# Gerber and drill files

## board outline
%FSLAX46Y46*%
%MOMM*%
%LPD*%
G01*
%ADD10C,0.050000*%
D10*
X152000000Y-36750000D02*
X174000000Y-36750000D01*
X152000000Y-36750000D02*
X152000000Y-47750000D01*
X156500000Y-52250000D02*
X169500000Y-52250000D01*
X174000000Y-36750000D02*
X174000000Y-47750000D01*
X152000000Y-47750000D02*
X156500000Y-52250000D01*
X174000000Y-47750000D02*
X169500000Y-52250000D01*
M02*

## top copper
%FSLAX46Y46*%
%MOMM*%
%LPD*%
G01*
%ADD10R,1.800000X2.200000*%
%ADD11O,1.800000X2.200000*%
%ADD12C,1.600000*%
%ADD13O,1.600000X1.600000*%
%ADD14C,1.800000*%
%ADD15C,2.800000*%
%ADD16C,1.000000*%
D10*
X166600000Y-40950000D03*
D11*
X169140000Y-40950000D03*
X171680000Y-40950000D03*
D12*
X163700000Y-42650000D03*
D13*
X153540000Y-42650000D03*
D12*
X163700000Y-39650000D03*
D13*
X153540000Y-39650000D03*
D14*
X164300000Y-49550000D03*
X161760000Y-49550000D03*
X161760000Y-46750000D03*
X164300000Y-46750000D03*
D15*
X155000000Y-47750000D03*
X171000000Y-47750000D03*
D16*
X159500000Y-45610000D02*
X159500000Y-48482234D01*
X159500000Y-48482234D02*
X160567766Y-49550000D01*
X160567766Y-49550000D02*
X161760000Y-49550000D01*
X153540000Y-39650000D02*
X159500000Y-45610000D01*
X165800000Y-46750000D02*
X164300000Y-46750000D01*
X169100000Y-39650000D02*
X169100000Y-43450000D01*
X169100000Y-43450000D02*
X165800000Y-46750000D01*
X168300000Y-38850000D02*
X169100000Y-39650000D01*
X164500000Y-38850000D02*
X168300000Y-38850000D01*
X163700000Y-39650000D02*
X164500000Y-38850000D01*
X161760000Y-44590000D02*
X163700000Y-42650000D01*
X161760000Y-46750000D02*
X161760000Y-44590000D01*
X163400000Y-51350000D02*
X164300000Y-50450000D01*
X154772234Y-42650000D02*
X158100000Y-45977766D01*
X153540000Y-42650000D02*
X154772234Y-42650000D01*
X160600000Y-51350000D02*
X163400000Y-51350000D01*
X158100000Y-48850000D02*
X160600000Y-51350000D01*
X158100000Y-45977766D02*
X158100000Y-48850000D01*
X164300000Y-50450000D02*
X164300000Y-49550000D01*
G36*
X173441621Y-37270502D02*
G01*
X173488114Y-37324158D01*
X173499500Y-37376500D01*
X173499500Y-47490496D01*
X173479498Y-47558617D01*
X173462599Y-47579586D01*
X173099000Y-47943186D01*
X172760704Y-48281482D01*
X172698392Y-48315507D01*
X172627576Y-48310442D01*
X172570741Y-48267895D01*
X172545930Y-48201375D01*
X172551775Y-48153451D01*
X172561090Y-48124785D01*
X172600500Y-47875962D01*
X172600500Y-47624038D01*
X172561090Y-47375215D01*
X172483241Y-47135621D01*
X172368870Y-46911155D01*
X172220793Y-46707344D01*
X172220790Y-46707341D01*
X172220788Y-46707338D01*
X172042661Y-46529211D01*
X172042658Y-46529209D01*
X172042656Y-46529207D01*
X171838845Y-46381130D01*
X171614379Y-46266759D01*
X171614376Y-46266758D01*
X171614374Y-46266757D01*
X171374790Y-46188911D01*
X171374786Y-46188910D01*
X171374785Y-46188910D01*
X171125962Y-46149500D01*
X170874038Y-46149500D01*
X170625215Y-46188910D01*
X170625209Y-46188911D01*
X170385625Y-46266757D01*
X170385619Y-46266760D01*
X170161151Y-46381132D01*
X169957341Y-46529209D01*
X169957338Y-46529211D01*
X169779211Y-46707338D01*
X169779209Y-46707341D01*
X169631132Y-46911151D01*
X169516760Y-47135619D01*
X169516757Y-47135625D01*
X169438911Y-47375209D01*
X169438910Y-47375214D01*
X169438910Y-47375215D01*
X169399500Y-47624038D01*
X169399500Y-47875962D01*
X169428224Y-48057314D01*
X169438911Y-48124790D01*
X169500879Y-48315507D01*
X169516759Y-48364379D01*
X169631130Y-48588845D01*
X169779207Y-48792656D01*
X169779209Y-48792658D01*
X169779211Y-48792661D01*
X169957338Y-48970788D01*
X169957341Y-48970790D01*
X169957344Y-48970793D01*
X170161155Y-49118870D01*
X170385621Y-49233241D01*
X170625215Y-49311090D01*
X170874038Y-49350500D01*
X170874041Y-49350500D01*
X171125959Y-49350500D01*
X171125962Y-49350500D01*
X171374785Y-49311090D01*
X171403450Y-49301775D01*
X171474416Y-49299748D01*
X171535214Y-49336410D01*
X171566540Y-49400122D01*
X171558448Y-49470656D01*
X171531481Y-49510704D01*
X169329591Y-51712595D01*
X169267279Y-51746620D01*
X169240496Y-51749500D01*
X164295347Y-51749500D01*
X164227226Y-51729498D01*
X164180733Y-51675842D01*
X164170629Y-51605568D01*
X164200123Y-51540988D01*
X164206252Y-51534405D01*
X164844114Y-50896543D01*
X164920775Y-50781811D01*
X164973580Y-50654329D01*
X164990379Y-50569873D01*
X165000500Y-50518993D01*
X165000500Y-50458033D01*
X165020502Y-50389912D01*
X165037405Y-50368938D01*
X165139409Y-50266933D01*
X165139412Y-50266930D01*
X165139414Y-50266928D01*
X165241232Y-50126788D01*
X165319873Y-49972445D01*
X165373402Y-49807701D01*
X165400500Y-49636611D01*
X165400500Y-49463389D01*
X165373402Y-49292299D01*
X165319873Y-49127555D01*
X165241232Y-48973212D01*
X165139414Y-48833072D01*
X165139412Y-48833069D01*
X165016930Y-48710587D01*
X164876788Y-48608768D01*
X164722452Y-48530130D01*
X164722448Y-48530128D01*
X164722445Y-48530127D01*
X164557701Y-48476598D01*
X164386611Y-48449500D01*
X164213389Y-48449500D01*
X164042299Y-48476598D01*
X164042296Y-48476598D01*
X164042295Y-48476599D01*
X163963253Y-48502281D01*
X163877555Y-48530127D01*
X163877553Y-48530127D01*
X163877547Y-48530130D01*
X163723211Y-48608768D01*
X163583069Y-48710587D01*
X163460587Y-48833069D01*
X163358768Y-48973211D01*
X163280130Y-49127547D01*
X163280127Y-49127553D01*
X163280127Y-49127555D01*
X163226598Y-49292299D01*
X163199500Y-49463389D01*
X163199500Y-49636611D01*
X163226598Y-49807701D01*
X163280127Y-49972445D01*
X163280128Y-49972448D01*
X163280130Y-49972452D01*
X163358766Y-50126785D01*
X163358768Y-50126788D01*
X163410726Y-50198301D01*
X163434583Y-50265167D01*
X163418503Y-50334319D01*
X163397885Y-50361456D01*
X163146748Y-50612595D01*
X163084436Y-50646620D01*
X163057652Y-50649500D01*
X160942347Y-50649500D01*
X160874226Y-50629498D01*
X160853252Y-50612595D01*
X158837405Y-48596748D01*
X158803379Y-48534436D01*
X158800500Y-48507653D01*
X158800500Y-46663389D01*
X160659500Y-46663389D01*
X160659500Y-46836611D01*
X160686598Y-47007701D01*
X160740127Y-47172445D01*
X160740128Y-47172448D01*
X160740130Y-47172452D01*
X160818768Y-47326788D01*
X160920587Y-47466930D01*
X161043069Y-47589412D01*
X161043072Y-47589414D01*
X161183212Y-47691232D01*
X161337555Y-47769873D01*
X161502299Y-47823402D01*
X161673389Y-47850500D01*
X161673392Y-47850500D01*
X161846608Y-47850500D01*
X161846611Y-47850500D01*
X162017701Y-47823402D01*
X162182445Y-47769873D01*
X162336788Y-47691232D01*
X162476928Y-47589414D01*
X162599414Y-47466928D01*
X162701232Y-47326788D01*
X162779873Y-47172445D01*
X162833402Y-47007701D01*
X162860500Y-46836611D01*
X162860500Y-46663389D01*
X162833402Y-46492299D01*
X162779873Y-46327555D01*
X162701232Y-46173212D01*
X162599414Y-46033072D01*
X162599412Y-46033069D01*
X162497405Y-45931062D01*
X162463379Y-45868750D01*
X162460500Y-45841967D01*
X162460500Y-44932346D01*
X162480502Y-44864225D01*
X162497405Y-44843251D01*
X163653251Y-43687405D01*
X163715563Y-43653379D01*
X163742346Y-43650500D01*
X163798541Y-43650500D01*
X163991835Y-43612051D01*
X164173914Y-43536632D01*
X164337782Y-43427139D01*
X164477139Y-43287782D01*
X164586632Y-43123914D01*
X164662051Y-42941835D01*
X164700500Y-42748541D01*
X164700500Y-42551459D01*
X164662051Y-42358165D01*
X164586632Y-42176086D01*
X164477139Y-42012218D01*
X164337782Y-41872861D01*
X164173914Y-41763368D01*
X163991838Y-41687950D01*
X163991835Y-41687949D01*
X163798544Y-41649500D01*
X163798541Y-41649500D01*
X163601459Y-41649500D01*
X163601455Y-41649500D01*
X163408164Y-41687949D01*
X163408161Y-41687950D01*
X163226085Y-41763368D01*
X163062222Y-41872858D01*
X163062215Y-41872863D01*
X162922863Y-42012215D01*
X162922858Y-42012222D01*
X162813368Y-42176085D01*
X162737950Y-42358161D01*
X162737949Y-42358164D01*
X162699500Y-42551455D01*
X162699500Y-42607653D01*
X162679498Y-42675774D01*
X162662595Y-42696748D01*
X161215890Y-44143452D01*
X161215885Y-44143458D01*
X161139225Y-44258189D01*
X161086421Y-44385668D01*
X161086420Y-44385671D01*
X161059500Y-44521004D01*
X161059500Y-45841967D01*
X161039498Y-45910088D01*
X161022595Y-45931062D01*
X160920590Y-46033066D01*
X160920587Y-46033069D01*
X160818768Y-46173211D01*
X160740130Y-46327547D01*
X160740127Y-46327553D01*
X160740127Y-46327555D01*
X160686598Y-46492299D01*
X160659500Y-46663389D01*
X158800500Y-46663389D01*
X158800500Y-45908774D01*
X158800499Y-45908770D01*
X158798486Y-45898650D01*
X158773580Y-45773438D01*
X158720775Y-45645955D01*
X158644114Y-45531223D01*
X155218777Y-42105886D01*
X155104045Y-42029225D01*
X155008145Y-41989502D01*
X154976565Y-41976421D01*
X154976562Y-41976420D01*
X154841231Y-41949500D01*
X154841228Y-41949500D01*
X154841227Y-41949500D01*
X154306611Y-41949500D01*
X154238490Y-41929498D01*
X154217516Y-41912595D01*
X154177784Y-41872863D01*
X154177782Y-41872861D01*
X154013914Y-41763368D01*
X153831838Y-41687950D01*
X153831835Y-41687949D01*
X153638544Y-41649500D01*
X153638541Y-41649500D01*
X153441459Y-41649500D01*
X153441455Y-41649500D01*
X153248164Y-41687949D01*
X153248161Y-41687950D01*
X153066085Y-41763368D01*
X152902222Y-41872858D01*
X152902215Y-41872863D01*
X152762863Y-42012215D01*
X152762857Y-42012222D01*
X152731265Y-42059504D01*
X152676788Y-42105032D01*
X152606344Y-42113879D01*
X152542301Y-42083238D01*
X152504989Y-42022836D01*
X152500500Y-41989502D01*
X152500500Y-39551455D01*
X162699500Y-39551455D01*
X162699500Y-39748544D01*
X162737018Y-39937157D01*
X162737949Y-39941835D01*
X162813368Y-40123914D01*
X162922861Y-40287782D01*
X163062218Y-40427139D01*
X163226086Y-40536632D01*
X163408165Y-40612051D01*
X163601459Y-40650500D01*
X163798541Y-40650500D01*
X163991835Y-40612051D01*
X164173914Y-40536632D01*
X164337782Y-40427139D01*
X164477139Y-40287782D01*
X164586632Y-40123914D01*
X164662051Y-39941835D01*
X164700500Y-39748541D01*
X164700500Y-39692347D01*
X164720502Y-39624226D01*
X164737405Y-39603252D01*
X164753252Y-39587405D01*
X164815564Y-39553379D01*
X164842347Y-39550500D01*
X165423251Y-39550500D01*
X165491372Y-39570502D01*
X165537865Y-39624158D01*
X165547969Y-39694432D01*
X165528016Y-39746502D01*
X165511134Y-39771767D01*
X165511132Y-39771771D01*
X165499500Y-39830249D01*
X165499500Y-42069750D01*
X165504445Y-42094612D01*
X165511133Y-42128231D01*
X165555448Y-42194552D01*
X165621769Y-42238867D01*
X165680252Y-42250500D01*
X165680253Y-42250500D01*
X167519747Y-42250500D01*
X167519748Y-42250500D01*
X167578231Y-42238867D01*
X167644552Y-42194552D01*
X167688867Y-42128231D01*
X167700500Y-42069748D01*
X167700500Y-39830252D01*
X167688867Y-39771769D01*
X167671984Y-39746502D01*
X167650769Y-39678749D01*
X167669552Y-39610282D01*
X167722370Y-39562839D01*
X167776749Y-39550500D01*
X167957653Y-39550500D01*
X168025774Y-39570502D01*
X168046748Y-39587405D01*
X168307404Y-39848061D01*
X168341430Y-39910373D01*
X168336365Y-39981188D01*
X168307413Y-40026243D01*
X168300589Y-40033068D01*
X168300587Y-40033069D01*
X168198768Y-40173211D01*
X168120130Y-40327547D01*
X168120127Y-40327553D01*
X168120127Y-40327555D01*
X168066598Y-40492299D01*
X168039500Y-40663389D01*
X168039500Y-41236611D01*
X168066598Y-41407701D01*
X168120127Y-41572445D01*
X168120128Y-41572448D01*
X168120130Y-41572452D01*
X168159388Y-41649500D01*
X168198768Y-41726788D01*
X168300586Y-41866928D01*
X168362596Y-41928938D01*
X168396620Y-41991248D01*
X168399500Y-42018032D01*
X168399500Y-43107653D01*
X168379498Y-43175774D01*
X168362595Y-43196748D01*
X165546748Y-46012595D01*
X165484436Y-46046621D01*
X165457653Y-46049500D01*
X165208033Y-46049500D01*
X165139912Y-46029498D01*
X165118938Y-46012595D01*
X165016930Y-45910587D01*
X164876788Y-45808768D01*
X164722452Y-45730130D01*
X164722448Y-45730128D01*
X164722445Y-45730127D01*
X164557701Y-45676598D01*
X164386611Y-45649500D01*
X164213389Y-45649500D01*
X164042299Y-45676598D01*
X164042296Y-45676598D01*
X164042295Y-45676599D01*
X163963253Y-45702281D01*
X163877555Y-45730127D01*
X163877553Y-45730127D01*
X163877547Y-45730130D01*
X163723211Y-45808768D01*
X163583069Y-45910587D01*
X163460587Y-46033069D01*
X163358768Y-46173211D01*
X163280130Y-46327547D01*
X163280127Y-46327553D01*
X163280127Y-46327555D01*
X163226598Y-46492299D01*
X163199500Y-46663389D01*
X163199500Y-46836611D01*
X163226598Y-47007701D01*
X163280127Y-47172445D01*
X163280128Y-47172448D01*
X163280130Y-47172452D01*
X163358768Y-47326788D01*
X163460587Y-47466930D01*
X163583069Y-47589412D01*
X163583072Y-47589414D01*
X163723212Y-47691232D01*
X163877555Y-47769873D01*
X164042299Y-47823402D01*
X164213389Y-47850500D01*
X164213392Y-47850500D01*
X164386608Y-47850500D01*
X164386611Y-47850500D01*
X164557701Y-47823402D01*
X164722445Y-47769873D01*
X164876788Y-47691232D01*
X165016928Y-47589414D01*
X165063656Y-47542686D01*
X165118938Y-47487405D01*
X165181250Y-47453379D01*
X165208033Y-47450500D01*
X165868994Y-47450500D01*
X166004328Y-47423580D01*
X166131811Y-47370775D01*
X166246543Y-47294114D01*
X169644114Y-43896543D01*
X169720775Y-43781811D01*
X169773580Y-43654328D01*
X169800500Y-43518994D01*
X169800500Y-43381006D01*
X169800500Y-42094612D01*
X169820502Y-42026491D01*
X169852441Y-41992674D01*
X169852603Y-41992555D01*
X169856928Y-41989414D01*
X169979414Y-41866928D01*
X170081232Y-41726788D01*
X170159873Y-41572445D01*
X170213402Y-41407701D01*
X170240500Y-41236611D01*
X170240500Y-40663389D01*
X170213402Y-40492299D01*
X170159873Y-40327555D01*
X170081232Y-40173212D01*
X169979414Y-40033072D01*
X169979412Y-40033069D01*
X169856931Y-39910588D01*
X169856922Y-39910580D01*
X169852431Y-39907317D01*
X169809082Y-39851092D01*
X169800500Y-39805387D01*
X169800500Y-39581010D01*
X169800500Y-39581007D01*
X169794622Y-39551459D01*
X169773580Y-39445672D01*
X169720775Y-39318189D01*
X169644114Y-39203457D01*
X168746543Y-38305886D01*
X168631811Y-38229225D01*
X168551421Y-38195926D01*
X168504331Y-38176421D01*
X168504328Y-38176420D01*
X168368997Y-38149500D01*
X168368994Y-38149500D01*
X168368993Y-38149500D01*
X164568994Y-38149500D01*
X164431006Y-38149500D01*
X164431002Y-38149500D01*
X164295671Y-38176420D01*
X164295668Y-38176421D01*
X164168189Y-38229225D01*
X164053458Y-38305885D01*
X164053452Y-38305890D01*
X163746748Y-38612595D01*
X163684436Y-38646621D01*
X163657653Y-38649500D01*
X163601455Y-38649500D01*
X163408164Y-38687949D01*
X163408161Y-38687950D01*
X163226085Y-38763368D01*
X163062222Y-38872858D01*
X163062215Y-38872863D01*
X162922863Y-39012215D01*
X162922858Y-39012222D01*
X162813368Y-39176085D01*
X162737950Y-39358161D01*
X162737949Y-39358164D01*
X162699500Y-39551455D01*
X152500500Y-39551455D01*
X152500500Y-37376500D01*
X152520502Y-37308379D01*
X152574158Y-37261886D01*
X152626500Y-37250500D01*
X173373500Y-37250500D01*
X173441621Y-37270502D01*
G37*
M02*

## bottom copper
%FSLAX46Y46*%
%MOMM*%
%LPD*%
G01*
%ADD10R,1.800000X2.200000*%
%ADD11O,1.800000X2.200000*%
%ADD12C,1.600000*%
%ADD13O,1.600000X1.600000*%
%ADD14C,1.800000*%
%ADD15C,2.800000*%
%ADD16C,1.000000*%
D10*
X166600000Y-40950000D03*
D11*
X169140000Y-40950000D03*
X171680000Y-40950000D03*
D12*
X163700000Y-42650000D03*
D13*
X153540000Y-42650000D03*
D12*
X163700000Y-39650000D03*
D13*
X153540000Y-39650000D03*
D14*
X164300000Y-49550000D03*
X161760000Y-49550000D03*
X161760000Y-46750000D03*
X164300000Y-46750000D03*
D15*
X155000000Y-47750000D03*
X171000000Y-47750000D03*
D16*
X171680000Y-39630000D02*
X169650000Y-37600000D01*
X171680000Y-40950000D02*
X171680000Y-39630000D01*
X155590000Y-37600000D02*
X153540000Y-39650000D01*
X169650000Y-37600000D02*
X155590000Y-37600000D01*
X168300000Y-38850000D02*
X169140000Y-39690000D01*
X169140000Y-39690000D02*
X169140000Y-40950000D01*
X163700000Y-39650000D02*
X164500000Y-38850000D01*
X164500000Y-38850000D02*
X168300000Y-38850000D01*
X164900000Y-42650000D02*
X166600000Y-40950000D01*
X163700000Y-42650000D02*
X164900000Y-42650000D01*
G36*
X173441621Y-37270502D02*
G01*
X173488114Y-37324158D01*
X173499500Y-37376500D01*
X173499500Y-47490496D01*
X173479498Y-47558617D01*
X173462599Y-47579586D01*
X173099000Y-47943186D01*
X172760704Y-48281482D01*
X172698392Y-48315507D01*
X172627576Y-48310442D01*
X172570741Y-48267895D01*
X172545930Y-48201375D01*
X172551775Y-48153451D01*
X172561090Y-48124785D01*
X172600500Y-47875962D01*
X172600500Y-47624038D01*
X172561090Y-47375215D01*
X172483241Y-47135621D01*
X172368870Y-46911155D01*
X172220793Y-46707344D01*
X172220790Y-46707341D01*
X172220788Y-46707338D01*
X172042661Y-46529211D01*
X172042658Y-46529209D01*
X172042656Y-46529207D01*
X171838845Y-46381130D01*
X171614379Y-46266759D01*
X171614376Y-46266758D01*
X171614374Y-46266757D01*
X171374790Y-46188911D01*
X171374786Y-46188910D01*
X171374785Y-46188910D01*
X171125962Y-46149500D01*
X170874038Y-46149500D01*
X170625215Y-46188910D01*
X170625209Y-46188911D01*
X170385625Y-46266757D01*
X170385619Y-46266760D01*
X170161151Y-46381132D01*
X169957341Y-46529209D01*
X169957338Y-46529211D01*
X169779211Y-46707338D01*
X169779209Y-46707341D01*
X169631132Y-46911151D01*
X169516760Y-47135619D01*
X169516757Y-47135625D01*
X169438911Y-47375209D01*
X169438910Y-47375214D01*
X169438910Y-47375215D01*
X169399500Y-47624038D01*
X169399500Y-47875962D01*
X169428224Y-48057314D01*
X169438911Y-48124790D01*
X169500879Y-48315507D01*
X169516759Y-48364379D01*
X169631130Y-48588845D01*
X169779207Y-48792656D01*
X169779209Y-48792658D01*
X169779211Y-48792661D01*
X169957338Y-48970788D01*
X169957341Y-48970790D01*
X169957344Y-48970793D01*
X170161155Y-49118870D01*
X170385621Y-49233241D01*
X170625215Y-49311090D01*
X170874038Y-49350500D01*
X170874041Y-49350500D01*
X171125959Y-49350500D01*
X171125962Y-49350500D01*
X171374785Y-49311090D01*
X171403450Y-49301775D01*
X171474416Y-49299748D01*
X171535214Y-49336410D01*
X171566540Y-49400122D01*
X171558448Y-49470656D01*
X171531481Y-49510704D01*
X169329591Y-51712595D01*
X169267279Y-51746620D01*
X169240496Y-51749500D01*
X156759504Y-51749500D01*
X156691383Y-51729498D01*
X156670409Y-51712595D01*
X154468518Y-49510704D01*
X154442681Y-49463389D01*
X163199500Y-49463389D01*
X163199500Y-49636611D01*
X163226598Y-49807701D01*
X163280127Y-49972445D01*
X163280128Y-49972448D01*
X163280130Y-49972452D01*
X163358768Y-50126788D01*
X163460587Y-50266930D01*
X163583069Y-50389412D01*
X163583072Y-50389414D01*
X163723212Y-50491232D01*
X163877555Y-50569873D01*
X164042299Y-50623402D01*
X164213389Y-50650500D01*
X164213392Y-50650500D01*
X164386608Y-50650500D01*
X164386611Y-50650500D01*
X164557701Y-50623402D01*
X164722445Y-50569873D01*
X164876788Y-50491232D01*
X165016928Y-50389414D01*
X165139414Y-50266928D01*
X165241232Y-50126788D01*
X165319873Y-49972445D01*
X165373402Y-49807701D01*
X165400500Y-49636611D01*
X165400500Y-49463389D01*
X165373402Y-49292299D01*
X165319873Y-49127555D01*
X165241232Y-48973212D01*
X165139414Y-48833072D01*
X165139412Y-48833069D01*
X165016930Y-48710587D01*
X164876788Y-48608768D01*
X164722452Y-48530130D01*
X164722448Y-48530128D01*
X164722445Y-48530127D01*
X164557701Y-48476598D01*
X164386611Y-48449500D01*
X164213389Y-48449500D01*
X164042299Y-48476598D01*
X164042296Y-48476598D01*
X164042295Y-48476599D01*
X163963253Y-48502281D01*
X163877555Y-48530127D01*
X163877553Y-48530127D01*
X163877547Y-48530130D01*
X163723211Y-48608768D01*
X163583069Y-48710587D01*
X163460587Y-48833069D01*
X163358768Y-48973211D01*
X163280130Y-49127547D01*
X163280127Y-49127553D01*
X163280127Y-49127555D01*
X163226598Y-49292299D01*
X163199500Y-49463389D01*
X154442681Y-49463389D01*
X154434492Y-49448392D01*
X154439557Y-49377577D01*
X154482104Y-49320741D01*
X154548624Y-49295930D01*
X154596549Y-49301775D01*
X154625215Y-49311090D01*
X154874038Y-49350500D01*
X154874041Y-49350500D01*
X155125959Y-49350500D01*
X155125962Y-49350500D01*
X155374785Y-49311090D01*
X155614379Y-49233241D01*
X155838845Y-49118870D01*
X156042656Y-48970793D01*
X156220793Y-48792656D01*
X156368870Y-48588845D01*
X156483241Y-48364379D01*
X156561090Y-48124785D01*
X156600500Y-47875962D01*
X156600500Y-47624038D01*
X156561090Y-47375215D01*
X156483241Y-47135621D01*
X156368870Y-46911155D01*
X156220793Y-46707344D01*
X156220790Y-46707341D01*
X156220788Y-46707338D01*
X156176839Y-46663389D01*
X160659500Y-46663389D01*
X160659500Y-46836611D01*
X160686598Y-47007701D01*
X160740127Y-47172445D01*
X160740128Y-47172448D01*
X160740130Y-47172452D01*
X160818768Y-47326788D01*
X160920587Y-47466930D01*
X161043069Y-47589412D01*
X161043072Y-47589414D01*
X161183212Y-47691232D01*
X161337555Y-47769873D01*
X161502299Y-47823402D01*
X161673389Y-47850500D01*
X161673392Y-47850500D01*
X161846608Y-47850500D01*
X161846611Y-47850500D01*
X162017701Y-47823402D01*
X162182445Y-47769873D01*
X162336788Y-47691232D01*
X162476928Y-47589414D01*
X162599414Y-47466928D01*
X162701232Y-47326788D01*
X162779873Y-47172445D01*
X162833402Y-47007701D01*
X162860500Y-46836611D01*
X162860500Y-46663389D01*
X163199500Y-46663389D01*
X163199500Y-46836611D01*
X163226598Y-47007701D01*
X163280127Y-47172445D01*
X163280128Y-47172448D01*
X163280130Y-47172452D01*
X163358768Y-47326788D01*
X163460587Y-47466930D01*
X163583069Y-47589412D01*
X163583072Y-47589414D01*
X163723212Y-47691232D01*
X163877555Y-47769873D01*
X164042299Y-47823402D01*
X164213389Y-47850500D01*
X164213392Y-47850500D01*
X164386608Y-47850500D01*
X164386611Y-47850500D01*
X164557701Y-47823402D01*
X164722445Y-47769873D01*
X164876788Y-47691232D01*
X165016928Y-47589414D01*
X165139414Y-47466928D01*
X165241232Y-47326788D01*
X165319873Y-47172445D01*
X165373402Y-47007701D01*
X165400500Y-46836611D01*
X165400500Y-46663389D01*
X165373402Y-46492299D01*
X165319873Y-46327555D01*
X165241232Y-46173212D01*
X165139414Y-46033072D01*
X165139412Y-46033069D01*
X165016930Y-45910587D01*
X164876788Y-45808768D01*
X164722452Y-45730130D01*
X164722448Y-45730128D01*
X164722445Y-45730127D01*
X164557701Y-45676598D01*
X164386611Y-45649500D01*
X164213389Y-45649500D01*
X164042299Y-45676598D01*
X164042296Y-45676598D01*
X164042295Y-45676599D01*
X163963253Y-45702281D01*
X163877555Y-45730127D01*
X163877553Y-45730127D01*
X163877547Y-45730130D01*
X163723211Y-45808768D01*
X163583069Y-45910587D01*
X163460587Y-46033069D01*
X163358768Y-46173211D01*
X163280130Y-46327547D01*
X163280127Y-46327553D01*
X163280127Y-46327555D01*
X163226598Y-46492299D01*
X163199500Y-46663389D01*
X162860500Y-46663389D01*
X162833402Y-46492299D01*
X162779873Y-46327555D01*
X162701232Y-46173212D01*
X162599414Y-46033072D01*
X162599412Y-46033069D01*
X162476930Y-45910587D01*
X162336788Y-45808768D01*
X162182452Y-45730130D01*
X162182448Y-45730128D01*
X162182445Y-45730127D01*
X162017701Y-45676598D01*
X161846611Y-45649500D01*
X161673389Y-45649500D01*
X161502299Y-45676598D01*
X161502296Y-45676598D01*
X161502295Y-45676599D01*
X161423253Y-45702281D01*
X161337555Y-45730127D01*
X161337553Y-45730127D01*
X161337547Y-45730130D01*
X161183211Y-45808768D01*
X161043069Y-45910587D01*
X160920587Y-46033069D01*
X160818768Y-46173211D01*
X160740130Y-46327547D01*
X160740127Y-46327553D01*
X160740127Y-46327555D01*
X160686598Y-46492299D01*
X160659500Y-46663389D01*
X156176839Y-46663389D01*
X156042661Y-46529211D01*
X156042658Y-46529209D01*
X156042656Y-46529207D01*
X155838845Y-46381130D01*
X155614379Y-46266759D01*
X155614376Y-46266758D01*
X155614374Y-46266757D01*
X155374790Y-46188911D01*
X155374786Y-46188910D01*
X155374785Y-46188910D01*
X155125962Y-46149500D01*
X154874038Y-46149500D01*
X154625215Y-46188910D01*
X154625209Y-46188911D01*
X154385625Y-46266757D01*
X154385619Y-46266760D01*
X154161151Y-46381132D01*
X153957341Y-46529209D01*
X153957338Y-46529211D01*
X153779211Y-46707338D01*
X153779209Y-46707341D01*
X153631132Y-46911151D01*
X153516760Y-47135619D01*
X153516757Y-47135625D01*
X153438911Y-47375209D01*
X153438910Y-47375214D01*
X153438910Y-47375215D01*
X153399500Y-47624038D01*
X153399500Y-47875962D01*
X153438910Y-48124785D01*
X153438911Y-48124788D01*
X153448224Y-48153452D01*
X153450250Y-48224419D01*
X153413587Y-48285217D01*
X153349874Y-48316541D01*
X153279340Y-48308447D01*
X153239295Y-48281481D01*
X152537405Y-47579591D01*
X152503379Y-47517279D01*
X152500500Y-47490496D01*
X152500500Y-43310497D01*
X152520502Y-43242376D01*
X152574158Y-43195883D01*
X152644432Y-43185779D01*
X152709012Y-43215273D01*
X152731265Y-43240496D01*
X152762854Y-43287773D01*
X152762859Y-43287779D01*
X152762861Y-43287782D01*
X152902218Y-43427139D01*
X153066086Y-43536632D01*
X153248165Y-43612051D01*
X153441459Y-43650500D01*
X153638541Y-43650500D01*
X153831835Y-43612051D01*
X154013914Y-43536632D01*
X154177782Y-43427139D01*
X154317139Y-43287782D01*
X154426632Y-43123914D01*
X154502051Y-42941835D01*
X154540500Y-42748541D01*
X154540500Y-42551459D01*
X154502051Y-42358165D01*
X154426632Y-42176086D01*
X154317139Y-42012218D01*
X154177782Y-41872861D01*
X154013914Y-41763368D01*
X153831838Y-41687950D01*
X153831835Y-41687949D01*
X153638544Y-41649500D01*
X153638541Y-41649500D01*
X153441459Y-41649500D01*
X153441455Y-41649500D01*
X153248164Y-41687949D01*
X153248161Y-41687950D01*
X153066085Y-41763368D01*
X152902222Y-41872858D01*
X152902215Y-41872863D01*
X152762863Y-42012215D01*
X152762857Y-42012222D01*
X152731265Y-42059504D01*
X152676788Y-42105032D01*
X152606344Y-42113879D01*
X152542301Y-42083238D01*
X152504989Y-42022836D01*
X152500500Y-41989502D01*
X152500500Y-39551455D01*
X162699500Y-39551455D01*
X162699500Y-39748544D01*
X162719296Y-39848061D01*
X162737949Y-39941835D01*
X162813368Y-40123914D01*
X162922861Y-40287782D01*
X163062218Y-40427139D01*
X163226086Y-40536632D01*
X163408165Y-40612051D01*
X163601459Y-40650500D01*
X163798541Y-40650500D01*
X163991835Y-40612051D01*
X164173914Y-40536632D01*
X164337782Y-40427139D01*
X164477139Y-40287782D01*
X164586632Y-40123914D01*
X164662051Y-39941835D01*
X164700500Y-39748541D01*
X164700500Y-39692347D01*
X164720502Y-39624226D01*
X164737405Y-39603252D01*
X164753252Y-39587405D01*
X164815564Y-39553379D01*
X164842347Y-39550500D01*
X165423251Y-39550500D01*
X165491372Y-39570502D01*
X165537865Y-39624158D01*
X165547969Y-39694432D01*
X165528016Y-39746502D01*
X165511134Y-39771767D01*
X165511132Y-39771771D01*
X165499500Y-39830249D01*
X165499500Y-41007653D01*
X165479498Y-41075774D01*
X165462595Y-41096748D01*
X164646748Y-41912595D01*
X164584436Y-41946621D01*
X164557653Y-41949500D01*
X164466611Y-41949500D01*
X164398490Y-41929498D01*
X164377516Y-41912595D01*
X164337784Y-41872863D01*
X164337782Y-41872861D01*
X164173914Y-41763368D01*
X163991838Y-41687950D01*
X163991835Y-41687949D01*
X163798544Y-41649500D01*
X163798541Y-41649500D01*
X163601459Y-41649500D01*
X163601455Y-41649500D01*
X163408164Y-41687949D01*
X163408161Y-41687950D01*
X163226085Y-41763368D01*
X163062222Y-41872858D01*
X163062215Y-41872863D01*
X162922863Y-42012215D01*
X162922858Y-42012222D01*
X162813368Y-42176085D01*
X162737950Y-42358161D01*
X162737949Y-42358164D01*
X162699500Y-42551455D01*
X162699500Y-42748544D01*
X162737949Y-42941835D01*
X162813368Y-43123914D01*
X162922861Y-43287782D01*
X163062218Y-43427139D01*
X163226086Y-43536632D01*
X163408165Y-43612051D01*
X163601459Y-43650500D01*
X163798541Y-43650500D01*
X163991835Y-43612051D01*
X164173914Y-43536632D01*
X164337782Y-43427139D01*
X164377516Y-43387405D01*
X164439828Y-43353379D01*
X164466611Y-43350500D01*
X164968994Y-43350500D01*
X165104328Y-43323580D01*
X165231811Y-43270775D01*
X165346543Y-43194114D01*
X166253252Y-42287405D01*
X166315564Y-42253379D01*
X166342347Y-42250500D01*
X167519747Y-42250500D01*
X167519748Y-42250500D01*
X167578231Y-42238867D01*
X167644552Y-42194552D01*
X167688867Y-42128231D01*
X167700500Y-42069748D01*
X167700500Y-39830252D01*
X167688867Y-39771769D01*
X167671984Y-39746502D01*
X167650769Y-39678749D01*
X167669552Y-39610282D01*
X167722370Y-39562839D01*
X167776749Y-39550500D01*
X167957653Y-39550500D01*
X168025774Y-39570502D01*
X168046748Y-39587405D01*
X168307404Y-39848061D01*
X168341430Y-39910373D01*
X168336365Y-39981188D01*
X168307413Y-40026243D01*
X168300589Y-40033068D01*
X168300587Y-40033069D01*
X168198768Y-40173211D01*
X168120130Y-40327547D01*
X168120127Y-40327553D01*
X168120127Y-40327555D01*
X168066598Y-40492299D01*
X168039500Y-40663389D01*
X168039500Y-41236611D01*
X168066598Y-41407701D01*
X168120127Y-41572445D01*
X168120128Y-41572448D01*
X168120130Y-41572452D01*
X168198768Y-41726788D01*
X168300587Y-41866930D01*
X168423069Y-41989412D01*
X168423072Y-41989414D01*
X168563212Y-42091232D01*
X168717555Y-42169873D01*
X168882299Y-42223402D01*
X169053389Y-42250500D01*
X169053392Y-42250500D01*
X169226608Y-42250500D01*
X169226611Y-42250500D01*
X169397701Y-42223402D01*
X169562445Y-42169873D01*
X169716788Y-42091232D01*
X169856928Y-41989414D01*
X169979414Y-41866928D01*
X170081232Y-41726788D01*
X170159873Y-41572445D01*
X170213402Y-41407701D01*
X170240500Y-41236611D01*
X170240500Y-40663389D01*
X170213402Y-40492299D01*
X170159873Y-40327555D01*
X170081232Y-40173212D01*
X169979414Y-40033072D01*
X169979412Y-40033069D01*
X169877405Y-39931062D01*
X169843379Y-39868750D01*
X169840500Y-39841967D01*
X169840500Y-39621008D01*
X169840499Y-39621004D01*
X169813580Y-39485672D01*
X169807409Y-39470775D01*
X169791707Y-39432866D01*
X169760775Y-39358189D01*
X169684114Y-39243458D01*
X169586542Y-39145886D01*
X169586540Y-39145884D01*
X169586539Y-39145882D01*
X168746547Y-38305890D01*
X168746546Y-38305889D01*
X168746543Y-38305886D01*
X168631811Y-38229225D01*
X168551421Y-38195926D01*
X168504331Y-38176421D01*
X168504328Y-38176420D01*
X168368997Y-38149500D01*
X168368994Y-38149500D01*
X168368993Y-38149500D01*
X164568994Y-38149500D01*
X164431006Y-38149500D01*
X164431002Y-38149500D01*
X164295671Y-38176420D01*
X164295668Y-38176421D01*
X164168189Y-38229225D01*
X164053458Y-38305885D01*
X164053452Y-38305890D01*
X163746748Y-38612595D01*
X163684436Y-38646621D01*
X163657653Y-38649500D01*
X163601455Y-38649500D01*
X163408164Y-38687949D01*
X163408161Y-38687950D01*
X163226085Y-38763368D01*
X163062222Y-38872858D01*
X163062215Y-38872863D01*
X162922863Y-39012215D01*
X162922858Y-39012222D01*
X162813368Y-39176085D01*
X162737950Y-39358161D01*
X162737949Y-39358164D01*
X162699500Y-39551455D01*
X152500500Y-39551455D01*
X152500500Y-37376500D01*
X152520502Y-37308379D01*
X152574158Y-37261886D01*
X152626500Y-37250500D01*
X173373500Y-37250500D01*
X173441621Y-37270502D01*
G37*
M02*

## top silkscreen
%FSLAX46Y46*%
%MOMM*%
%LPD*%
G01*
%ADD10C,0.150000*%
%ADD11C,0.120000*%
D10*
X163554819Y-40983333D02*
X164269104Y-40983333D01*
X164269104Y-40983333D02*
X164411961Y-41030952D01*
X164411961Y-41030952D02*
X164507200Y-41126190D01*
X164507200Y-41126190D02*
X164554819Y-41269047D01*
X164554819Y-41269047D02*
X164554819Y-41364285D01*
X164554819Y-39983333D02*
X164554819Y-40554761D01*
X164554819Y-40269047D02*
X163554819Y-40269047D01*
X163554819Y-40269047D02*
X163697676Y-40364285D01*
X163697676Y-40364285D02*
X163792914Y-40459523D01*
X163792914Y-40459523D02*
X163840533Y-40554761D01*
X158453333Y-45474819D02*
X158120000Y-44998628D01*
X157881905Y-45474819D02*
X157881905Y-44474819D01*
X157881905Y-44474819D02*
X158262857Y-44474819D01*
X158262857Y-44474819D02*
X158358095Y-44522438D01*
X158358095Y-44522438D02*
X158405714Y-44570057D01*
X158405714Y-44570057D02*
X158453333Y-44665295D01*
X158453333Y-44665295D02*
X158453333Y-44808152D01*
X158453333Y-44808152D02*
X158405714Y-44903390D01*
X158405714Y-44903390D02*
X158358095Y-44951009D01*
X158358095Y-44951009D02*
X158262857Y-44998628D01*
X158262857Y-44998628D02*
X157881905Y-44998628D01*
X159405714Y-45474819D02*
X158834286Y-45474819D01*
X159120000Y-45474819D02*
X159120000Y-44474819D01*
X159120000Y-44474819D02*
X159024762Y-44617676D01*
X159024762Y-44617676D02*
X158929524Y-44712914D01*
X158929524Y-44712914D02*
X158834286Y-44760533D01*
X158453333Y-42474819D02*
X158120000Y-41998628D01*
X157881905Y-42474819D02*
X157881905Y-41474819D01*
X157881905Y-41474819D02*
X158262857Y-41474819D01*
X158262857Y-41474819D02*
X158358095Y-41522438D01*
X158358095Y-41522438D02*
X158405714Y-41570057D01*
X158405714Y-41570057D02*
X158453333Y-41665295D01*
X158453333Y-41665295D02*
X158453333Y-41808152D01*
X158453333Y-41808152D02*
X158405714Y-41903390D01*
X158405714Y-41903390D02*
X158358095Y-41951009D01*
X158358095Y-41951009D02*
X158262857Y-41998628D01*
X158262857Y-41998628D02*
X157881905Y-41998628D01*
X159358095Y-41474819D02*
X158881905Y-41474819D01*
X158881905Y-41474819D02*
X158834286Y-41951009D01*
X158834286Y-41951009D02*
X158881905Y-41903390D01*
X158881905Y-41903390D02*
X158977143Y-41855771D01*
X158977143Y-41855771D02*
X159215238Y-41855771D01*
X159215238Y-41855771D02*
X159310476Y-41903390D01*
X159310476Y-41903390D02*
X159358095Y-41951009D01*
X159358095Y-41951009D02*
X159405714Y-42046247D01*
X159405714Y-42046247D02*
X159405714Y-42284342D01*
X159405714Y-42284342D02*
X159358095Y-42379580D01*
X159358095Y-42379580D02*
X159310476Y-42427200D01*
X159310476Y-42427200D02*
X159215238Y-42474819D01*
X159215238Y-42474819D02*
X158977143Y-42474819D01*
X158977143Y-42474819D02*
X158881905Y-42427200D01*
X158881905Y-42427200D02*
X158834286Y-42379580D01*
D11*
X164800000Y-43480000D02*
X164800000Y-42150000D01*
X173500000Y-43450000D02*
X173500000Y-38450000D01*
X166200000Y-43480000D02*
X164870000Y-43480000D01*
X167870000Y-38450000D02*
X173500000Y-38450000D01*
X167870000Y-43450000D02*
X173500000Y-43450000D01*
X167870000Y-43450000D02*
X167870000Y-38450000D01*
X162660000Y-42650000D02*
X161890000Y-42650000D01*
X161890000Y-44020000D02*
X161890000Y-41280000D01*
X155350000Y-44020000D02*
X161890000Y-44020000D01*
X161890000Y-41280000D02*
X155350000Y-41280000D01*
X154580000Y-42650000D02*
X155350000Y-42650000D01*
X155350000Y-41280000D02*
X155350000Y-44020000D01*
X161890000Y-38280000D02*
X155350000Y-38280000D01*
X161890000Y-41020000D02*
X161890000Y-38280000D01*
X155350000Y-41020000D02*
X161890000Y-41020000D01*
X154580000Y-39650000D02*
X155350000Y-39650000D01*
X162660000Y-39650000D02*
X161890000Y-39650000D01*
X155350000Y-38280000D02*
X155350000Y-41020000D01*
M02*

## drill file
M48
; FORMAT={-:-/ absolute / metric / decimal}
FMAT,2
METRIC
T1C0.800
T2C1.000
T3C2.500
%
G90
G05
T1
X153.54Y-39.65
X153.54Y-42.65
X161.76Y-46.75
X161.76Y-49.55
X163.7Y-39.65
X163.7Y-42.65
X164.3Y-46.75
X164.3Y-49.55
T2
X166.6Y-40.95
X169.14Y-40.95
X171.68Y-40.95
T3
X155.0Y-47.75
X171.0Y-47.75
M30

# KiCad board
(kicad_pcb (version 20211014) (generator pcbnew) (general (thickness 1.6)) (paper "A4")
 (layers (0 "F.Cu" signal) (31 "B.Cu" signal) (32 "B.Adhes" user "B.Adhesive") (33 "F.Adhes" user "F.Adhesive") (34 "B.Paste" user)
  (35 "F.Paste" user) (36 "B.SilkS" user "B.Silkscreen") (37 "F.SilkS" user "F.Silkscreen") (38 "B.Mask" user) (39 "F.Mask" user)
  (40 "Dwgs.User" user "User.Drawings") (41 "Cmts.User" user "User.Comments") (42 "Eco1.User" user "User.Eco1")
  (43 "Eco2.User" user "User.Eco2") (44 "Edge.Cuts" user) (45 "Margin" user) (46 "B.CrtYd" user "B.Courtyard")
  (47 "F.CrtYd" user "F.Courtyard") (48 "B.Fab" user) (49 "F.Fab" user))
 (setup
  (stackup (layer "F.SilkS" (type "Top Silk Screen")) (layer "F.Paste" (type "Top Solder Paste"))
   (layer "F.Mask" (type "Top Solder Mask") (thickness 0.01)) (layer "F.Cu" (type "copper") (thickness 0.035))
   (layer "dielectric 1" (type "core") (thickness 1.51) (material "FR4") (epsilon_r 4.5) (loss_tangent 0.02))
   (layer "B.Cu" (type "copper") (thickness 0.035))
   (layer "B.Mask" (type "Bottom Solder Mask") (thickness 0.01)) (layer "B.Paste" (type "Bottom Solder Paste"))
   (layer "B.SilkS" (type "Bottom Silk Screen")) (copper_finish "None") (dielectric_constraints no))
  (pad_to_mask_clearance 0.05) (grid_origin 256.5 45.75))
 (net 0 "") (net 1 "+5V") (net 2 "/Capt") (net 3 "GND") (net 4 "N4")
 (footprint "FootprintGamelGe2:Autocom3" (layer "F.Cu") (at 166.6 40.95 90)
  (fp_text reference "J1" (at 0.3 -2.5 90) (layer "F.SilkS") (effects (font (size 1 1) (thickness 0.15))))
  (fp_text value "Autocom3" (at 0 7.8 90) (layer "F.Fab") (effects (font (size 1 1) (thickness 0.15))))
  (fp_line (start -2.53 -1.8) (end -1.2 -1.8) (layer "F.SilkS") (width 0.12))
  (fp_line (start -2.5 6.9) (end 2.5 6.9) (layer "F.SilkS") (width 0.12))
  (fp_line (start -2.53 -0.4) (end -2.53 -1.73) (layer "F.SilkS") (width 0.12))
  (fp_line (start 2.5 1.27) (end 2.5 6.9) (layer "F.SilkS") (width 0.12))
  (fp_line (start -2.5 1.27) (end -2.5 6.9) (layer "F.SilkS") (width 0.12))
  (fp_line (start -2.5 1.27) (end 2.5 1.27) (layer "F.SilkS") (width 0.12))
  (pad "1" thru_hole rect locked (at 0 0 90) (size 2.2 1.8) (drill 1) (layers *.Cu *.Mask) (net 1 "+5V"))
  (pad "2" thru_hole oval locked (at 0 2.54 90) (size 2.2 1.8) (drill 1) (layers *.Cu *.Mask) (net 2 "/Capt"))
  (pad "3" thru_hole oval locked (at 0 5.08 90) (size 2.2 1.8) (drill 1) (layers *.Cu *.Mask) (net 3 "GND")))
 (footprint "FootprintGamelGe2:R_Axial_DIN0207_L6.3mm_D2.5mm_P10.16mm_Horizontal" (layer "F.Cu") (at 163.7 42.65 180)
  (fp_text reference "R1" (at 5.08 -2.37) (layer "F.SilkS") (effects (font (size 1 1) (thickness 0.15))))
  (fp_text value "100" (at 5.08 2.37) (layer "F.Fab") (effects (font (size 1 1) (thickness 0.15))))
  (fp_line (start 1.04 0) (end 1.81 0) (layer "F.SilkS") (width 0.12))
  (fp_line (start 1.81 -1.37) (end 1.81 1.37) (layer "F.SilkS") (width 0.12))
  (fp_line (start 8.35 -1.37) (end 1.81 -1.37) (layer "F.SilkS") (width 0.12))
  (fp_line (start 1.81 1.37) (end 8.35 1.37) (layer "F.SilkS") (width 0.12))
  (fp_line (start 9.12 0) (end 8.35 0) (layer "F.SilkS") (width 0.12))
  (fp_line (start 8.35 1.37) (end 8.35 -1.37) (layer "F.SilkS") (width 0.12))
  (pad "1" thru_hole circle locked (at 0 0 180) (size 1.6 1.6) (drill 0.8) (layers *.Cu *.Mask) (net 1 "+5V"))
  (pad "2" thru_hole oval locked (at 10.16 0 180) (size 1.6 1.6) (drill 0.8) (layers *.Cu *.Mask) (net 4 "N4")))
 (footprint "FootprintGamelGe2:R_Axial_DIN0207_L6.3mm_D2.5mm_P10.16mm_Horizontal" (layer "F.Cu") (at 163.7 39.65 180)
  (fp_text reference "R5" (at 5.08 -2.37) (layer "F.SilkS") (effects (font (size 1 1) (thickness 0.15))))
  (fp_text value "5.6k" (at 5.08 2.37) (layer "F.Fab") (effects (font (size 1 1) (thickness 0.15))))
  (fp_line (start 1.81 1.37) (end 8.35 1.37) (layer "F.SilkS") (width 0.12))
  (fp_line (start 1.81 -1.37) (end 1.81 1.37) (layer "F.SilkS") (width 0.12))
  (fp_line (start 8.35 -1.37) (end 1.81 -1.37) (layer "F.SilkS") (width 0.12))
  (fp_line (start 9.12 0) (end 8.35 0) (layer "F.SilkS") (width 0.12))
  (fp_line (start 1.04 0) (end 1.81 0) (layer "F.SilkS") (width 0.12))
  (fp_line (start 8.35 1.37) (end 8.35 -1.37) (layer "F.SilkS") (width 0.12))
  (pad "1" thru_hole circle locked (at 0 0 180) (size 1.6 1.6) (drill 0.8) (layers *.Cu *.Mask) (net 2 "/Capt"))
  (pad "2" thru_hole oval locked (at 10.16 0 180) (size 1.6 1.6) (drill 0.8) (layers *.Cu *.Mask) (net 3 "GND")))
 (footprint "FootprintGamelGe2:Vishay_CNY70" (layer "B.Cu") (at 164.3 49.55 90)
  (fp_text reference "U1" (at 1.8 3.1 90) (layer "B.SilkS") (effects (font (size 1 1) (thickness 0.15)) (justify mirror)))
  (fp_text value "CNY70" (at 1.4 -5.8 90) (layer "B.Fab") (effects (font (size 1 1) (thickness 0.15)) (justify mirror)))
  (pad "1" thru_hole circle locked (at 0 0 90) (size 1.8 1.8) (drill 0.8) (layers *.Cu *.Mask) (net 4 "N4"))
  (pad "2" thru_hole circle locked (at 0 -2.54 90) (size 1.8 1.8) (drill 0.8) (layers *.Cu *.Mask) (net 3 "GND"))
  (pad "3" thru_hole circle locked (at 2.8 -2.54 90) (size 1.8 1.8) (drill 0.8) (layers *.Cu *.Mask) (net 1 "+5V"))
  (pad "4" thru_hole circle locked (at 2.8 0 90) (size 1.8 1.8) (drill 0.8) (layers *.Cu *.Mask) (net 2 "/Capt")))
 (gr_line (start 152 36.75) (end 174 36.75) (layer "Edge.Cuts") (width 0.05))
 (gr_line (start 152 36.75) (end 152 47.75) (layer "Edge.Cuts") (width 0.05))
 (gr_line (start 156.5 52.25) (end 169.5 52.25) (layer "Edge.Cuts") (width 0.05))
 (gr_line (start 174 36.75) (end 174 47.75) (layer "Edge.Cuts") (width 0.05))
 (gr_line (start 152 47.75) (end 156.5 52.25) (layer "Edge.Cuts") (width 0.05))
 (gr_line (start 174 47.75) (end 169.5 52.25) (layer "Edge.Cuts") (width 0.05))
 (via (at 155 47.75) (size 2.8) (drill 2.5) (layers "F.Cu" "B.Cu") (free) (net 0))
 (via (at 171 47.75) (size 2.8) (drill 2.5) (layers "F.Cu" "B.Cu") (free) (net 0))
 (segment (start 159.5 45.61) (end 159.5 48.482234) (width 1) (layer "F.Cu") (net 3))
 (segment (start 159.5 48.482234) (end 160.567766 49.55) (width 1) (layer "F.Cu") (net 3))
 (segment (start 160.567766 49.55) (end 161.76 49.55) (width 1) (layer "F.Cu") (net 3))
 (segment (start 153.54 39.65) (end 159.5 45.61) (width 1) (layer "F.Cu") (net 3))
 (segment (start 171.68 39.63) (end 169.65 37.6) (width 1) (layer "B.Cu") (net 3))
 (segment (start 171.68 40.95) (end 171.68 39.63) (width 1) (layer "B.Cu") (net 3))
 (segment (start 155.59 37.6) (end 153.54 39.65) (width 1) (layer "B.Cu") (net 3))
 (segment (start 169.65 37.6) (end 155.59 37.6) (width 1) (layer "B.Cu") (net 3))
 (segment (start 165.8 46.75) (end 164.3 46.75) (width 1) (layer "F.Cu") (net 2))
 (segment (start 169.1 39.65) (end 169.1 43.45) (width 1) (layer "F.Cu") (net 2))
 (segment (start 169.1 43.45) (end 165.8 46.75) (width 1) (layer "F.Cu") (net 2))
 (segment (start 168.3 38.85) (end 169.1 39.65) (width 1) (layer "F.Cu") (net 2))
 (segment (start 164.5 38.85) (end 168.3 38.85) (width 1) (layer "F.Cu") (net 2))
 (segment (start 163.7 39.65) (end 164.5 38.85) (width 1) (layer "F.Cu") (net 2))
 (segment (start 168.3 38.85) (end 169.14 39.69) (width 1) (layer "B.Cu") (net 2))
 (segment (start 169.14 39.69) (end 169.14 40.95) (width 1) (layer "B.Cu") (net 2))
 (segment (start 163.7 39.65) (end 164.5 38.85) (width 1) (layer "B.Cu") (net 2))
 (segment (start 164.5 38.85) (end 168.3 38.85) (width 1) (layer "B.Cu") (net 2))
 (segment (start 161.76 44.59) (end 163.7 42.65) (width 1) (layer "F.Cu") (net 1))
 (segment (start 161.76 46.75) (end 161.76 44.59) (width 1) (layer "F.Cu") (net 1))
 (segment (start 164.9 42.65) (end 166.6 40.95) (width 1) (layer "B.Cu") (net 1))
 (segment (start 163.7 42.65) (end 164.9 42.65) (width 1) (layer "B.Cu") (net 1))
 (segment (start 163.4 51.35) (end 164.3 50.45) (width 1) (layer "F.Cu") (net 4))
 (segment (start 154.772234 42.65) (end 158.1 45.977766) (width 1) (layer "F.Cu") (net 4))
 (segment (start 153.54 42.65) (end 154.772234 42.65) (width 1) (layer "F.Cu") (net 4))
 (segment (start 160.6 51.35) (end 163.4 51.35) (width 1) (layer "F.Cu") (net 4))
 (segment (start 158.1 48.85) (end 160.6 51.35) (width 1) (layer "F.Cu") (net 4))
 (segment (start 158.1 45.977766) (end 158.1 48.85) (width 1) (layer "F.Cu") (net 4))
 (segment (start 164.3 50.45) (end 164.3 49.55) (width 1) (layer "F.Cu") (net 4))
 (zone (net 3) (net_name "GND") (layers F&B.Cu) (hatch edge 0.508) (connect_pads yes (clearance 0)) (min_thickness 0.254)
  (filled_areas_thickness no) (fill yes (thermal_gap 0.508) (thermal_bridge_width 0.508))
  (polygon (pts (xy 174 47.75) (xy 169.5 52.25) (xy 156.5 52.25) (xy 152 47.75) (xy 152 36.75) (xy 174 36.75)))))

